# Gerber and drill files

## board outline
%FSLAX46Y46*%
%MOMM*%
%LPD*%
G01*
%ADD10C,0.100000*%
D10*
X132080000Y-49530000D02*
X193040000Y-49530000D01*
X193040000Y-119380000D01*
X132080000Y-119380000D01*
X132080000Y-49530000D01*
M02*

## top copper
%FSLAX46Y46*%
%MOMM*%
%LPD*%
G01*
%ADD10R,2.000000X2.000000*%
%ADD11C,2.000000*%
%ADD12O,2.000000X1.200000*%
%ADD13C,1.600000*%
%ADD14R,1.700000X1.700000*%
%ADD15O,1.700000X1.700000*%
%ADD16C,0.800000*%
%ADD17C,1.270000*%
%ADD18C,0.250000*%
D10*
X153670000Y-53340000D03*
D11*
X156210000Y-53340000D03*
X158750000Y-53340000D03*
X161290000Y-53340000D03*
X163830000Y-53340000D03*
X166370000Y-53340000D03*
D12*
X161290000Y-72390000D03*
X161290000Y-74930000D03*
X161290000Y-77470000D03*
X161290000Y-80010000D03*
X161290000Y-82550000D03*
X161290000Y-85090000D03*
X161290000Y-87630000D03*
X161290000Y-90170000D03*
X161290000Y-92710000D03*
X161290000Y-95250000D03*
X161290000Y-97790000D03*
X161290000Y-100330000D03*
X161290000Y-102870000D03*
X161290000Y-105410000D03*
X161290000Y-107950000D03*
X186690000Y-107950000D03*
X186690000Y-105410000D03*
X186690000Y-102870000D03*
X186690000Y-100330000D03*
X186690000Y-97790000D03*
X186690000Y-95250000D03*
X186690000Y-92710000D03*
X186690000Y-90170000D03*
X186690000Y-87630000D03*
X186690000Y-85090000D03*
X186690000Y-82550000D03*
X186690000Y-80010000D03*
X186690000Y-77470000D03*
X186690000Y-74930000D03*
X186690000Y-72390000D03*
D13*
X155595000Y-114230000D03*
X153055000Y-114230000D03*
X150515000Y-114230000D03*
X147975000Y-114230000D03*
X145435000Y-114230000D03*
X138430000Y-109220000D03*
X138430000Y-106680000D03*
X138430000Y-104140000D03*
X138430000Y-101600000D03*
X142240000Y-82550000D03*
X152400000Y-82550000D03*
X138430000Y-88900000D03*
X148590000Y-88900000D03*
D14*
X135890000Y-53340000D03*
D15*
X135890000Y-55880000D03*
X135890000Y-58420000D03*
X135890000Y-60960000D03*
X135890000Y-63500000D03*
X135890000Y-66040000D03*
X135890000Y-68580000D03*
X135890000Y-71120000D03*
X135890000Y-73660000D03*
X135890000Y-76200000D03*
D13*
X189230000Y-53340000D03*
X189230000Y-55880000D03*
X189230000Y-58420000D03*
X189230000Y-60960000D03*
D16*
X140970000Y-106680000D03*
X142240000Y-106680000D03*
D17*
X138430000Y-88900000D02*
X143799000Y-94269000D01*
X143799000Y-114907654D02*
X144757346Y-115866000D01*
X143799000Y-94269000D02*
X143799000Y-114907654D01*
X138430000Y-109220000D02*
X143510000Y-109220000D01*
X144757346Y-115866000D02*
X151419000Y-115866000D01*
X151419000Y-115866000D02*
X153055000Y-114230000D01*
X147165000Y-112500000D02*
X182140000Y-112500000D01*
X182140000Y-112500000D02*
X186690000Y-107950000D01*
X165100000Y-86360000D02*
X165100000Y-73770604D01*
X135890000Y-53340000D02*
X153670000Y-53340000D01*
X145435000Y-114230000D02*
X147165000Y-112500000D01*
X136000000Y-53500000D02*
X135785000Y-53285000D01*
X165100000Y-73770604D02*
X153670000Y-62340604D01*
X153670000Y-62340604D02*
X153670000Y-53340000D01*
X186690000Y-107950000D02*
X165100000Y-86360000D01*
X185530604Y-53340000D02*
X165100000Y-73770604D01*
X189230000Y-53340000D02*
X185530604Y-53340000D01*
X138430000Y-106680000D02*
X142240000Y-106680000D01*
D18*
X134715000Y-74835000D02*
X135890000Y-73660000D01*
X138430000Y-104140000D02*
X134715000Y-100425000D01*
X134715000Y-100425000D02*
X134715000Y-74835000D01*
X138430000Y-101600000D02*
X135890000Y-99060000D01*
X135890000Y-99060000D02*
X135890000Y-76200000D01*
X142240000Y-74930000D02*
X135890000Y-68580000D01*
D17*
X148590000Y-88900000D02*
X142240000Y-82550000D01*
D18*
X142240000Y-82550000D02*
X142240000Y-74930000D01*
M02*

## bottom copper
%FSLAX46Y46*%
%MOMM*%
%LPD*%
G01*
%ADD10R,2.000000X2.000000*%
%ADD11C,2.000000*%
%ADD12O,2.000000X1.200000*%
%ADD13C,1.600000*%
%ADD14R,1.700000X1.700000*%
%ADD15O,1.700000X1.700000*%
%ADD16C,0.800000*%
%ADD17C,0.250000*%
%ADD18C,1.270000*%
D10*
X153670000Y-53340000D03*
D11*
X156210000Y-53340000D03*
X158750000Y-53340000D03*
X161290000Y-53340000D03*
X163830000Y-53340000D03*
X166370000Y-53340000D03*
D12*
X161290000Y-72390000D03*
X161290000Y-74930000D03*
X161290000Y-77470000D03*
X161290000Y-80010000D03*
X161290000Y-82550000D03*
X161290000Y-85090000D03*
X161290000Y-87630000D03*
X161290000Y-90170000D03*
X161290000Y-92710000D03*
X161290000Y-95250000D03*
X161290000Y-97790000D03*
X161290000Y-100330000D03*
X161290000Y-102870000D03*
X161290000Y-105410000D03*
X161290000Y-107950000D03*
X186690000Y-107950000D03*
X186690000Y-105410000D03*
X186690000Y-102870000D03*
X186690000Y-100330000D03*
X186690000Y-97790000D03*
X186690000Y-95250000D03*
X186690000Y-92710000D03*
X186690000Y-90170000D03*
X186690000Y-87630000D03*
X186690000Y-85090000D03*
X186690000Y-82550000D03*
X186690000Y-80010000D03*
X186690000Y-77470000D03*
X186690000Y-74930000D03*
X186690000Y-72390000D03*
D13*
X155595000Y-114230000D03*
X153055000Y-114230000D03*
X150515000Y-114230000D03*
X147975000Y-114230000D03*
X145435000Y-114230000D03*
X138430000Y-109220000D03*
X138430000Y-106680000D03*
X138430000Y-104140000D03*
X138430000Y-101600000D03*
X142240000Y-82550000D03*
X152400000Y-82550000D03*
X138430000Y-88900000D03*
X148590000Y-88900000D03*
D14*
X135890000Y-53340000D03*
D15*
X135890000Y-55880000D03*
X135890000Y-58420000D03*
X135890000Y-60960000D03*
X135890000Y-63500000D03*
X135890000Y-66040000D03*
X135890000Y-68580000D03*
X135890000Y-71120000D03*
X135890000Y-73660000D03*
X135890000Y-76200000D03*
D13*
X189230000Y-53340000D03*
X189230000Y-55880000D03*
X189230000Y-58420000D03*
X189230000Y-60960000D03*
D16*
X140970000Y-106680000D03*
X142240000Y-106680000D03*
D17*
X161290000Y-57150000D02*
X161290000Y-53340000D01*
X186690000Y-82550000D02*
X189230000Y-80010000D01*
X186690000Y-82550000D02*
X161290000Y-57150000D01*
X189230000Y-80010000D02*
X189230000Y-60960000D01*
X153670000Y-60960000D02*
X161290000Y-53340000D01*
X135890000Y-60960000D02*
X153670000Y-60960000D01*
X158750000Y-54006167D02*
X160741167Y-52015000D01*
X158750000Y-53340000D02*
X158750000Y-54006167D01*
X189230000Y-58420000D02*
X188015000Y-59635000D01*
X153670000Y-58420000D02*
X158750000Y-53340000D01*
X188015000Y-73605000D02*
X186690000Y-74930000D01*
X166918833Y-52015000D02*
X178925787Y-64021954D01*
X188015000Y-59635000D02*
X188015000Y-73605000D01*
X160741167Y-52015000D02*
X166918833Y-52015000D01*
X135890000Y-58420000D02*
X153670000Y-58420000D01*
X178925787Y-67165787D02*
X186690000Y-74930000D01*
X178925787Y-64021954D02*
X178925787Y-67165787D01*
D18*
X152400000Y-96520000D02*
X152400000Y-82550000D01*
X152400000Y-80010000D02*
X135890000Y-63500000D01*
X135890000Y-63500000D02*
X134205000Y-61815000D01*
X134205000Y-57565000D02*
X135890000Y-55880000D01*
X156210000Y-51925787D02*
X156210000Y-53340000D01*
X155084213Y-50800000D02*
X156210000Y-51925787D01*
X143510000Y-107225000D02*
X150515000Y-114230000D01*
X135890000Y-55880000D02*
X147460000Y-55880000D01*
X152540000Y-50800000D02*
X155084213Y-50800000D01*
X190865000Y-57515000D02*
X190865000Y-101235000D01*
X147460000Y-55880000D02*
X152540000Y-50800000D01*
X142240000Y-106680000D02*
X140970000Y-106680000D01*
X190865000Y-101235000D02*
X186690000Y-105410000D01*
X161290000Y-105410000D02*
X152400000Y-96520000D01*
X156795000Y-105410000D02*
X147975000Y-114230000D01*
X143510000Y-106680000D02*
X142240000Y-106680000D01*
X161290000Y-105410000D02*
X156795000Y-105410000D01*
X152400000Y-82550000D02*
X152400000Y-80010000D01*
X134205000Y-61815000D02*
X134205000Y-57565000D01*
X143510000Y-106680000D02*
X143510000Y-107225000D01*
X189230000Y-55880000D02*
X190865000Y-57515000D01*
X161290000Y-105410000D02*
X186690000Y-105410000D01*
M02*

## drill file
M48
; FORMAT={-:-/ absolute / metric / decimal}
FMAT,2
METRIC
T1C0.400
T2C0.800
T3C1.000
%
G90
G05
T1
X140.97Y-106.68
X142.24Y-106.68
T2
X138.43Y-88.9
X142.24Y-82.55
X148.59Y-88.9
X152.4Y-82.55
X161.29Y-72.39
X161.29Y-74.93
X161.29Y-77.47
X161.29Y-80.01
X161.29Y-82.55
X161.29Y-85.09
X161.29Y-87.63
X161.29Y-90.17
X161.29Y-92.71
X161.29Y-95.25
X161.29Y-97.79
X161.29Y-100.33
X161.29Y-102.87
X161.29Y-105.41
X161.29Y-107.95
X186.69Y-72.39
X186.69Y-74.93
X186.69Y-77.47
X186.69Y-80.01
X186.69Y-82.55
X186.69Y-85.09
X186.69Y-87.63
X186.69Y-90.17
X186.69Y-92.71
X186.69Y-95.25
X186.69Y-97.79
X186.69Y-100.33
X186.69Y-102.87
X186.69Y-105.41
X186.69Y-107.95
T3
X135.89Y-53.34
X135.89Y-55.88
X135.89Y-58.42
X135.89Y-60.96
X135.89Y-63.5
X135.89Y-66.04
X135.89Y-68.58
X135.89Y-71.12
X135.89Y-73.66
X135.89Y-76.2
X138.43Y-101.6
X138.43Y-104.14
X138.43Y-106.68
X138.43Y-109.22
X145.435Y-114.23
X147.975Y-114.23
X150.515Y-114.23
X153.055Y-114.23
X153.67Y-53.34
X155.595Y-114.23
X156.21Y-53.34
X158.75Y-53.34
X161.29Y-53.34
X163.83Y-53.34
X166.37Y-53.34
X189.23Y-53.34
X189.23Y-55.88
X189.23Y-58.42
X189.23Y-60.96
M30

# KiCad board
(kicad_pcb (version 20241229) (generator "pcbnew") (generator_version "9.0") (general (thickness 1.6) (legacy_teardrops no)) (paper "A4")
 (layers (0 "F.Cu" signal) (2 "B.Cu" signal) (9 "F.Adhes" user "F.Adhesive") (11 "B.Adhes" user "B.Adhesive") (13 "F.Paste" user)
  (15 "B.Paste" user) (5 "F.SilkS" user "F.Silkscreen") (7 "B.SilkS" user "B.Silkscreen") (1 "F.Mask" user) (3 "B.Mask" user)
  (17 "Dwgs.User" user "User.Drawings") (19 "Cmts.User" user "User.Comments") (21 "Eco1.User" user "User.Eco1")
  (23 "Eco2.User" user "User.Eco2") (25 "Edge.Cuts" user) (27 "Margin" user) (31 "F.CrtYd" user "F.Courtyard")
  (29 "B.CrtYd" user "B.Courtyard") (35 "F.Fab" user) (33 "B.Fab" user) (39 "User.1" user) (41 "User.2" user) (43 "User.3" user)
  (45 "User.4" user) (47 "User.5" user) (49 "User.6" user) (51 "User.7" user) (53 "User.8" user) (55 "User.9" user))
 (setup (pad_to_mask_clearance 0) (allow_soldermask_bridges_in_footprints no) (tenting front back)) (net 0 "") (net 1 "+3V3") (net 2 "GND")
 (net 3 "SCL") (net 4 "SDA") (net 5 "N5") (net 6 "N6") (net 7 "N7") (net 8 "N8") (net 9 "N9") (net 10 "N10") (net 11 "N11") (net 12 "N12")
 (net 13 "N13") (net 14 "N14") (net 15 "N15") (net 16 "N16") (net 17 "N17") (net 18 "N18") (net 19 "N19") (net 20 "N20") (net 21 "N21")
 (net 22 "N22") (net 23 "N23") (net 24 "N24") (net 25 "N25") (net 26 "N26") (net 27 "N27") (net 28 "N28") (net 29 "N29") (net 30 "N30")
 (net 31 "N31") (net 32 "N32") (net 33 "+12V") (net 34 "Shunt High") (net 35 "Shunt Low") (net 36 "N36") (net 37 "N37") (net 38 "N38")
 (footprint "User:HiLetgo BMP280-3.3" (layer "F.Cu") (at 153.67 53.34 90)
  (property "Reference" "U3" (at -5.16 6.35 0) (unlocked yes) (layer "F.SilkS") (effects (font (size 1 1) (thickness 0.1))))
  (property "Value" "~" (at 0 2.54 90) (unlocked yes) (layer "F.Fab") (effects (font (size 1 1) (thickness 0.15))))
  (pad "1" thru_hole rect (at 0 0 90) (size 2 2) (drill 1) (layers "*.Cu" "*.Mask") (remove_unused_layers no) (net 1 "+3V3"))
  (pad "2" thru_hole circle (at 0 2.54 90) (size 2 2) (drill 1) (layers "*.Cu" "*.Mask") (remove_unused_layers no) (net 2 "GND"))
  (pad "3" thru_hole circle (at 0 5.08 90) (size 2 2) (drill 1) (layers "*.Cu" "*.Mask") (remove_unused_layers no) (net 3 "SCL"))
  (pad "4" thru_hole circle (at 0 7.62 90) (size 2 2) (drill 1) (layers "*.Cu" "*.Mask") (remove_unused_layers no) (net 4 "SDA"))
  (pad "5" thru_hole circle (at 0 10.16 90) (size 2 2) (drill 1) (layers "*.Cu" "*.Mask") (remove_unused_layers no) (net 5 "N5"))
  (pad "6" thru_hole circle (at 0 12.7 90) (size 2 2) (drill 1) (layers "*.Cu" "*.Mask") (remove_unused_layers no) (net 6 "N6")))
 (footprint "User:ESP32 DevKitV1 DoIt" (layer "F.Cu") (at 158.75 69.85)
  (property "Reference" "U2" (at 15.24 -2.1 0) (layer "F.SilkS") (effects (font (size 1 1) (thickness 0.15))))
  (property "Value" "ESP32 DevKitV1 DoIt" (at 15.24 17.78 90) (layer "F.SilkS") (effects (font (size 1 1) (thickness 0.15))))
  (pad "1" thru_hole oval (at 2.54 2.54 270) (size 1.2 2) (drill 0.8) (layers "*.Cu" "*.Mask") (remove_unused_layers no) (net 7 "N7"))
  (pad "2" thru_hole oval (at 2.54 5.08 270) (size 1.2 2) (drill 0.8) (layers "*.Cu" "*.Mask") (remove_unused_layers no) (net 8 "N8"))
  (pad "3" thru_hole oval (at 2.54 7.62 270) (size 1.2 2) (drill 0.8) (layers "*.Cu" "*.Mask") (remove_unused_layers no) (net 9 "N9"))
  (pad "4" thru_hole oval (at 2.54 10.16 270) (size 1.2 2) (drill 0.8) (layers "*.Cu" "*.Mask") (remove_unused_layers no) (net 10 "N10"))
  (pad "5" thru_hole oval (at 2.54 12.7 270) (size 1.2 2) (drill 0.8) (layers "*.Cu" "*.Mask") (remove_unused_layers no) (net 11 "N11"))
  (pad "6" thru_hole oval (at 2.54 15.24 270) (size 1.2 2) (drill 0.8) (layers "*.Cu" "*.Mask") (remove_unused_layers no) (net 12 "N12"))
  (pad "7" thru_hole oval (at 2.54 17.78 270) (size 1.2 2) (drill 0.8) (layers "*.Cu" "*.Mask") (remove_unused_layers no) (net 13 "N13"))
  (pad "8" thru_hole oval (at 2.54 20.32 270) (size 1.2 2) (drill 0.8) (layers "*.Cu" "*.Mask") (remove_unused_layers no) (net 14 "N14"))
  (pad "9" thru_hole oval (at 2.54 22.86 270) (size 1.2 2) (drill 0.8) (layers "*.Cu" "*.Mask") (remove_unused_layers no) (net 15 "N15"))
  (pad "10" thru_hole oval (at 2.54 25.4 270) (size 1.2 2) (drill 0.8) (layers "*.Cu" "*.Mask") (remove_unused_layers no) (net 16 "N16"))
  (pad "11" thru_hole oval (at 2.54 27.94 270) (size 1.2 2) (drill 0.8) (layers "*.Cu" "*.Mask") (remove_unused_layers no) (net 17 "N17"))
  (pad "12" thru_hole oval (at 2.54 30.48 270) (size 1.2 2) (drill 0.8) (layers "*.Cu" "*.Mask") (remove_unused_layers no) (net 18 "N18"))
  (pad "13" thru_hole oval (at 2.54 33.02 270) (size 1.2 2) (drill 0.8) (layers "*.Cu" "*.Mask") (remove_unused_layers no) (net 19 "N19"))
  (pad "14" thru_hole oval (at 2.54 35.56 270) (size 1.2 2) (drill 0.8) (layers "*.Cu" "*.Mask") (remove_unused_layers no) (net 2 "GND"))
  (pad "15" thru_hole oval (at 2.54 38.1 270) (size 1.2 2) (drill 0.8) (layers "*.Cu" "*.Mask") (remove_unused_layers no) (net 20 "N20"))
  (pad "16" thru_hole oval (at 27.94 38.1 270) (size 1.2 2) (drill 0.8) (layers "*.Cu" "*.Mask") (remove_unused_layers no) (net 1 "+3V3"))
  (pad "17" thru_hole oval (at 27.94 35.56 270) (size 1.2 2) (drill 0.8) (layers "*.Cu" "*.Mask") (remove_unused_layers no) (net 2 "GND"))
  (pad "18" thru_hole oval (at 27.94 33.02 270) (size 1.2 2) (drill 0.8) (layers "*.Cu" "*.Mask") (remove_unused_layers no) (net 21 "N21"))
  (pad "19" thru_hole oval (at 27.94 30.48 270) (size 1.2 2) (drill 0.8) (layers "*.Cu" "*.Mask") (remove_unused_layers no) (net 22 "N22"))
  (pad "20" thru_hole oval (at 27.94 27.94 270) (size 1.2 2) (drill 0.8) (layers "*.Cu" "*.Mask") (remove_unused_layers no) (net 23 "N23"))
  (pad "21" thru_hole oval (at 27.94 25.4 270) (size 1.2 2) (drill 0.8) (layers "*.Cu" "*.Mask") (remove_unused_layers no) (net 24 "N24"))
  (pad "22" thru_hole oval (at 27.94 22.86 270) (size 1.2 2) (drill 0.8) (layers "*.Cu" "*.Mask") (remove_unused_layers no) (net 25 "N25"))
  (pad "23" thru_hole oval (at 27.94 20.32 270) (size 1.2 2) (drill 0.8) (layers "*.Cu" "*.Mask") (remove_unused_layers no) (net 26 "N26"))
  (pad "24" thru_hole oval (at 27.94 17.78 270) (size 1.2 2) (drill 0.8) (layers "*.Cu" "*.Mask") (remove_unused_layers no) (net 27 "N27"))
  (pad "25" thru_hole oval (at 27.94 15.24 270) (size 1.2 2) (drill 0.8) (layers "*.Cu" "*.Mask") (remove_unused_layers no) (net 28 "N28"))
  (pad "26" thru_hole oval (at 27.94 12.7 270) (size 1.2 2) (drill 0.8) (layers "*.Cu" "*.Mask") (remove_unused_layers no) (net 4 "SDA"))
  (pad "27" thru_hole oval (at 27.94 10.16 270) (size 1.2 2) (drill 0.8) (layers "*.Cu" "*.Mask") (remove_unused_layers no) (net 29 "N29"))
  (pad "28" thru_hole oval (at 27.94 7.62 270) (size 1.2 2) (drill 0.8) (layers "*.Cu" "*.Mask") (remove_unused_layers no) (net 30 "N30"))
  (pad "29" thru_hole oval (at 27.94 5.08 270) (size 1.2 2) (drill 0.8) (layers "*.Cu" "*.Mask") (remove_unused_layers no) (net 3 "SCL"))
  (pad "30" thru_hole oval (at 27.94 2.54 270) (size 1.2 2) (drill 0.8) (layers "*.Cu" "*.Mask") (remove_unused_layers no) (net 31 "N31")))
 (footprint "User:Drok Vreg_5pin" (layer "F.Cu") (at 152 113 -90)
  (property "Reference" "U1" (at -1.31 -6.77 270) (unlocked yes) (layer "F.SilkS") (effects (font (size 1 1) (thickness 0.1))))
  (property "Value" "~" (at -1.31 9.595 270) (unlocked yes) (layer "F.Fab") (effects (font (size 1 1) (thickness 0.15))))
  (pad "1" thru_hole circle (at 1.23 -3.595 180) (size 1.6 1.6) (drill 1) (layers "*.Cu" "*.Mask") (remove_unused_layers no) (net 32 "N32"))
  (pad "2" thru_hole circle (at 1.23 -1.055 180) (size 1.6 1.6) (drill 1) (layers "*.Cu" "*.Mask") (remove_unused_layers no) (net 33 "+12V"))
  (pad "3" thru_hole circle (at 1.23 1.485 180) (size 1.6 1.6) (drill 1) (layers "*.Cu" "*.Mask") (remove_unused_layers no) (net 2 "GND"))
  (pad "4" thru_hole circle (at 1.23 4.025 180) (size 1.6 1.6) (drill 1) (layers "*.Cu" "*.Mask") (remove_unused_layers no) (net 2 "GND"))
  (pad "5" thru_hole circle (at 1.23 6.565 180) (size 1.6 1.6) (drill 1) (layers "*.Cu" "*.Mask") (remove_unused_layers no) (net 1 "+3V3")))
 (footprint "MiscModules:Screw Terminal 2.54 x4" (layer "F.Cu") (at 140.97 96.52 180)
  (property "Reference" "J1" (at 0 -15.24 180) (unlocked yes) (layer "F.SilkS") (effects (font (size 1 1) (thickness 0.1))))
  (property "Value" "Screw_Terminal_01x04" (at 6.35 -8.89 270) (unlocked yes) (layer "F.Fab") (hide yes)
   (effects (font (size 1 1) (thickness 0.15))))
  (pad "1" thru_hole circle (at 2.54 -12.7 90) (size 1.6 1.6) (drill 1) (layers "*.Cu" "*.Mask") (remove_unused_layers no) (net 33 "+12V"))
  (pad "2" thru_hole circle (at 2.54 -10.16 90) (size 1.6 1.6) (drill 1) (layers "*.Cu" "*.Mask") (remove_unused_layers no) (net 2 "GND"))
  (pad "3" thru_hole circle (at 2.54 -7.62 90) (size 1.6 1.6) (drill 1) (layers "*.Cu" "*.Mask") (remove_unused_layers no)
   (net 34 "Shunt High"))
  (pad "4" thru_hole circle (at 2.54 -5.08 90) (size 1.6 1.6) (drill 1) (layers "*.Cu" "*.Mask") (remove_unused_layers no)
   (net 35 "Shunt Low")))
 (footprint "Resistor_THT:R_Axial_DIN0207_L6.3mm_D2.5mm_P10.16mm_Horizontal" (layer "F.Cu") (at 142.24 82.55)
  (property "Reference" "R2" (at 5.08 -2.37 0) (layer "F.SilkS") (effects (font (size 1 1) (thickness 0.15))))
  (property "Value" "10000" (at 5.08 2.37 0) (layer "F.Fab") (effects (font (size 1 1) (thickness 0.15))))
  (pad "1" thru_hole circle (at 0 0) (size 1.6 1.6) (drill 0.8) (layers "*.Cu" "*.Mask") (remove_unused_layers no) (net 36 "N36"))
  (pad "2" thru_hole circle (at 10.16 0) (size 1.6 1.6) (drill 0.8) (layers "*.Cu" "*.Mask") (remove_unused_layers no) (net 2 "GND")))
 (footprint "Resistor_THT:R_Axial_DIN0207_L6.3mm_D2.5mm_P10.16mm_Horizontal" (layer "F.Cu") (at 138.43 88.9)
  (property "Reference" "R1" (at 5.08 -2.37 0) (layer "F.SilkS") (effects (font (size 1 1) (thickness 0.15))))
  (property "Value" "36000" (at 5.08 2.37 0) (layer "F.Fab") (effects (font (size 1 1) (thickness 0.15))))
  (pad "1" thru_hole circle (at 0 0) (size 1.6 1.6) (drill 0.8) (layers "*.Cu" "*.Mask") (remove_unused_layers no) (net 33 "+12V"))
  (pad "2" thru_hole circle (at 10.16 0) (size 1.6 1.6) (drill 0.8) (layers "*.Cu" "*.Mask") (remove_unused_layers no) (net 36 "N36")))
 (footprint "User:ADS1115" (layer "F.Cu") (at 135.89 53.34)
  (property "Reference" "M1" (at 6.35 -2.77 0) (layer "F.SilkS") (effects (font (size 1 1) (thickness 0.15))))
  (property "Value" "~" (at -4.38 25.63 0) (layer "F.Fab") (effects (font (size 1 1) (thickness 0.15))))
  (pad "1" thru_hole rect (at 0 0) (size 1.7 1.7) (drill 1) (layers "*.Cu" "*.Mask") (remove_unused_layers no) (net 1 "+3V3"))
  (pad "2" thru_hole oval (at 0 2.54) (size 1.7 1.7) (drill 1) (layers "*.Cu" "*.Mask") (remove_unused_layers no) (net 2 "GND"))
  (pad "3" thru_hole oval (at 0 5.08) (size 1.7 1.7) (drill 1) (layers "*.Cu" "*.Mask") (remove_unused_layers no) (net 3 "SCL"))
  (pad "4" thru_hole oval (at 0 7.62) (size 1.7 1.7) (drill 1) (layers "*.Cu" "*.Mask") (remove_unused_layers no) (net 4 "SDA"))
  (pad "5" thru_hole oval (at 0 10.16) (size 1.7 1.7) (drill 1) (layers "*.Cu" "*.Mask") (remove_unused_layers no) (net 2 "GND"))
  (pad "6" thru_hole oval (at 0 12.7) (size 1.7 1.7) (drill 1) (layers "*.Cu" "*.Mask") (remove_unused_layers no) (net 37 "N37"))
  (pad "7" thru_hole oval (at 0 15.24) (size 1.7 1.7) (drill 1) (layers "*.Cu" "*.Mask") (remove_unused_layers no) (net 36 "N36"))
  (pad "8" thru_hole oval (at 0 17.78) (size 1.7 1.7) (drill 1) (layers "*.Cu" "*.Mask") (remove_unused_layers no) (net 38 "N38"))
  (pad "9" thru_hole oval (at 0 20.32) (size 1.7 1.7) (drill 1) (layers "*.Cu" "*.Mask") (remove_unused_layers no) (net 34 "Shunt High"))
  (pad "10" thru_hole oval (at 0 22.86) (size 1.7 1.7) (drill 1) (layers "*.Cu" "*.Mask") (remove_unused_layers no) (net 35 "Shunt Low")))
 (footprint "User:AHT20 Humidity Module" (layer "F.Cu") (at 186.69 57.15)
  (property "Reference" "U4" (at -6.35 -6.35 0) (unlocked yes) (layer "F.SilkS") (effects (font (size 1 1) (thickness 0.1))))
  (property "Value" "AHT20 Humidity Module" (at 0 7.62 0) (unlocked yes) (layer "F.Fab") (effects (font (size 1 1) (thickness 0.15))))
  (pad "1" thru_hole circle (at 2.54 -3.81 270) (size 1.6 1.6) (drill 1) (layers "*.Cu" "*.Mask") (remove_unused_layers no) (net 1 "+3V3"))
  (pad "2" thru_hole circle (at 2.54 -1.27 270) (size 1.6 1.6) (drill 1) (layers "*.Cu" "*.Mask") (remove_unused_layers no) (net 2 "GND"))
  (pad "3" thru_hole circle (at 2.54 1.27 270) (size 1.6 1.6) (drill 1) (layers "*.Cu" "*.Mask") (remove_unused_layers no) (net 3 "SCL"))
  (pad "4" thru_hole circle (at 2.54 3.81 270) (size 1.6 1.6) (drill 1) (layers "*.Cu" "*.Mask") (remove_unused_layers no) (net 4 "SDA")))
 (gr_rect (start 132.08 49.53) (end 193.04 119.38) (stroke (width 0.1) (type default)) (fill no) (layer "Edge.Cuts"))
 (segment (start 138.43 88.9) (end 143.799 94.269) (width 1.27) (layer "F.Cu") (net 33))
 (segment (start 143.799 114.907654) (end 144.757346 115.866) (width 1.27) (layer "F.Cu") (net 33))
 (segment (start 143.799 94.269) (end 143.799 114.907654) (width 1.27) (layer "F.Cu") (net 33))
 (segment (start 138.43 109.22) (end 143.51 109.22) (width 1.27) (layer "F.Cu") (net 33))
 (segment (start 144.757346 115.866) (end 151.419 115.866) (width 1.27) (layer "F.Cu") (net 33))
 (segment (start 151.419 115.866) (end 153.055 114.23) (width 1.27) (layer "F.Cu") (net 33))
 (segment (start 147.165 112.5) (end 182.14 112.5) (width 1.27) (layer "F.Cu") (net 1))
 (segment (start 182.14 112.5) (end 186.69 107.95) (width 1.27) (layer "F.Cu") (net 1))
 (segment (start 165.1 86.36) (end 165.1 73.770604) (width 1.27) (layer "F.Cu") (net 1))
 (segment (start 135.89 53.34) (end 153.67 53.34) (width 1.27) (layer "F.Cu") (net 1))
 (segment (start 145.435 114.23) (end 147.165 112.5) (width 1.27) (layer "F.Cu") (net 1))
 (segment (start 136 53.5) (end 135.785 53.285) (width 1.27) (layer "F.Cu") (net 1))
 (segment (start 165.1 73.770604) (end 153.67 62.340604) (width 1.27) (layer "F.Cu") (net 1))
 (segment (start 153.67 62.340604) (end 153.67 53.34) (width 1.27) (layer "F.Cu") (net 1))
 (segment (start 186.69 107.95) (end 165.1 86.36) (width 1.27) (layer "F.Cu") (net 1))
 (segment (start 185.530604 53.34) (end 165.1 73.770604) (width 1.27) (layer "F.Cu") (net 1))
 (segment (start 189.23 53.34) (end 185.530604 53.34) (width 1.27) (layer "F.Cu") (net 1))
 (segment (start 161.29 57.15) (end 161.29 53.34) (width 0.25) (layer "B.Cu") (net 4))
 (segment (start 186.69 82.55) (end 189.23 80.01) (width 0.25) (layer "B.Cu") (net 4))
 (segment (start 186.69 82.55) (end 161.29 57.15) (width 0.25) (layer "B.Cu") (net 4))
 (segment (start 189.23 80.01) (end 189.23 60.96) (width 0.25) (layer "B.Cu") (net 4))
 (segment (start 153.67 60.96) (end 161.29 53.34) (width 0.25) (layer "B.Cu") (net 4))
 (segment (start 135.89 60.96) (end 153.67 60.96) (width 0.25) (layer "B.Cu") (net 4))
 (segment (start 158.75 54.006167) (end 160.741167 52.015) (width 0.25) (layer "B.Cu") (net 3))
 (segment (start 158.75 53.34) (end 158.75 54.006167) (width 0.25) (layer "B.Cu") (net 3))
 (segment (start 189.23 58.42) (end 188.015 59.635) (width 0.25) (layer "B.Cu") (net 3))
 (segment (start 153.67 58.42) (end 158.75 53.34) (width 0.25) (layer "B.Cu") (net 3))
 (segment (start 188.015 73.605) (end 186.69 74.93) (width 0.25) (layer "B.Cu") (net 3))
 (segment (start 166.918833 52.015) (end 178.925787 64.021954) (width 0.25) (layer "B.Cu") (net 3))
 (segment (start 188.015 59.635) (end 188.015 73.605) (width 0.25) (layer "B.Cu") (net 3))
 (segment (start 160.741167 52.015) (end 166.918833 52.015) (width 0.25) (layer "B.Cu") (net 3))
 (segment (start 135.89 58.42) (end 153.67 58.42) (width 0.25) (layer "B.Cu") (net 3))
 (segment (start 178.925787 67.165787) (end 186.69 74.93) (width 0.25) (layer "B.Cu") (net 3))
 (segment (start 178.925787 64.021954) (end 178.925787 67.165787) (width 0.25) (layer "B.Cu") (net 3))
 (segment (start 138.43 106.68) (end 142.24 106.68) (width 1.27) (layer "F.Cu") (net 2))
 (via (at 140.97 106.68) (size 0.8) (drill 0.4) (layers "F.Cu" "B.Cu") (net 2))
 (via (at 142.24 106.68) (size 0.8) (drill 0.4) (layers "F.Cu" "B.Cu") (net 2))
 (segment (start 152.4 96.52) (end 152.4 82.55) (width 1.27) (layer "B.Cu") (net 2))
 (segment (start 152.4 80.01) (end 135.89 63.5) (width 1.27) (layer "B.Cu") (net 2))
 (segment (start 135.89 63.5) (end 134.205 61.815) (width 1.27) (layer "B.Cu") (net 2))
 (segment (start 134.205 57.565) (end 135.89 55.88) (width 1.27) (layer "B.Cu") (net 2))
 (segment (start 156.21 51.925787) (end 156.21 53.34) (width 1.27) (layer "B.Cu") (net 2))
 (segment (start 155.084213 50.8) (end 156.21 51.925787) (width 1.27) (layer "B.Cu") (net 2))
 (segment (start 143.51 107.225) (end 150.515 114.23) (width 1.27) (layer "B.Cu") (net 2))
 (segment (start 135.89 55.88) (end 147.46 55.88) (width 1.27) (layer "B.Cu") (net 2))
 (segment (start 152.54 50.8) (end 155.084213 50.8) (width 1.27) (layer "B.Cu") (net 2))
 (segment (start 190.865 57.515) (end 190.865 101.235) (width 1.27) (layer "B.Cu") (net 2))
 (segment (start 147.46 55.88) (end 152.54 50.8) (width 1.27) (layer "B.Cu") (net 2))
 (segment (start 142.24 106.68) (end 140.97 106.68) (width 1.27) (layer "B.Cu") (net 2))
 (segment (start 190.865 101.235) (end 186.69 105.41) (width 1.27) (layer "B.Cu") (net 2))
 (segment (start 161.29 105.41) (end 152.4 96.52) (width 1.27) (layer "B.Cu") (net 2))
 (segment (start 156.795 105.41) (end 147.975 114.23) (width 1.27) (layer "B.Cu") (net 2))
 (segment (start 143.51 106.68) (end 142.24 106.68) (width 1.27) (layer "B.Cu") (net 2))
 (segment (start 161.29 105.41) (end 156.795 105.41) (width 1.27) (layer "B.Cu") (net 2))
 (segment (start 152.4 82.55) (end 152.4 80.01) (width 1.27) (layer "B.Cu") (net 2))
 (segment (start 134.205 61.815) (end 134.205 57.565) (width 1.27) (layer "B.Cu") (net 2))
 (segment (start 143.51 106.68) (end 143.51 107.225) (width 1.27) (layer "B.Cu") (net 2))
 (segment (start 189.23 55.88) (end 190.865 57.515) (width 1.27) (layer "B.Cu") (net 2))
 (segment (start 161.29 105.41) (end 186.69 105.41) (width 1.27) (layer "B.Cu") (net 2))
 (segment (start 134.715 74.835) (end 135.89 73.66) (width 0.25) (layer "F.Cu") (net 34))
 (segment (start 138.43 104.14) (end 134.715 100.425) (width 0.25) (layer "F.Cu") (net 34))
 (segment (start 134.715 100.425) (end 134.715 74.835) (width 0.25) (layer "F.Cu") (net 34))
 (segment (start 138.43 101.6) (end 135.89 99.06) (width 0.25) (layer "F.Cu") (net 35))
 (segment (start 135.89 99.06) (end 135.89 76.2) (width 0.25) (layer "F.Cu") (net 35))
 (segment (start 142.24 74.93) (end 135.89 68.58) (width 0.25) (layer "F.Cu") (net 36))
 (segment (start 148.59 88.9) (end 142.24 82.55) (width 1.27) (layer "F.Cu") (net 36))
 (segment (start 142.24 82.55) (end 142.24 74.93) (width 0.25) (layer "F.Cu") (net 36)))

